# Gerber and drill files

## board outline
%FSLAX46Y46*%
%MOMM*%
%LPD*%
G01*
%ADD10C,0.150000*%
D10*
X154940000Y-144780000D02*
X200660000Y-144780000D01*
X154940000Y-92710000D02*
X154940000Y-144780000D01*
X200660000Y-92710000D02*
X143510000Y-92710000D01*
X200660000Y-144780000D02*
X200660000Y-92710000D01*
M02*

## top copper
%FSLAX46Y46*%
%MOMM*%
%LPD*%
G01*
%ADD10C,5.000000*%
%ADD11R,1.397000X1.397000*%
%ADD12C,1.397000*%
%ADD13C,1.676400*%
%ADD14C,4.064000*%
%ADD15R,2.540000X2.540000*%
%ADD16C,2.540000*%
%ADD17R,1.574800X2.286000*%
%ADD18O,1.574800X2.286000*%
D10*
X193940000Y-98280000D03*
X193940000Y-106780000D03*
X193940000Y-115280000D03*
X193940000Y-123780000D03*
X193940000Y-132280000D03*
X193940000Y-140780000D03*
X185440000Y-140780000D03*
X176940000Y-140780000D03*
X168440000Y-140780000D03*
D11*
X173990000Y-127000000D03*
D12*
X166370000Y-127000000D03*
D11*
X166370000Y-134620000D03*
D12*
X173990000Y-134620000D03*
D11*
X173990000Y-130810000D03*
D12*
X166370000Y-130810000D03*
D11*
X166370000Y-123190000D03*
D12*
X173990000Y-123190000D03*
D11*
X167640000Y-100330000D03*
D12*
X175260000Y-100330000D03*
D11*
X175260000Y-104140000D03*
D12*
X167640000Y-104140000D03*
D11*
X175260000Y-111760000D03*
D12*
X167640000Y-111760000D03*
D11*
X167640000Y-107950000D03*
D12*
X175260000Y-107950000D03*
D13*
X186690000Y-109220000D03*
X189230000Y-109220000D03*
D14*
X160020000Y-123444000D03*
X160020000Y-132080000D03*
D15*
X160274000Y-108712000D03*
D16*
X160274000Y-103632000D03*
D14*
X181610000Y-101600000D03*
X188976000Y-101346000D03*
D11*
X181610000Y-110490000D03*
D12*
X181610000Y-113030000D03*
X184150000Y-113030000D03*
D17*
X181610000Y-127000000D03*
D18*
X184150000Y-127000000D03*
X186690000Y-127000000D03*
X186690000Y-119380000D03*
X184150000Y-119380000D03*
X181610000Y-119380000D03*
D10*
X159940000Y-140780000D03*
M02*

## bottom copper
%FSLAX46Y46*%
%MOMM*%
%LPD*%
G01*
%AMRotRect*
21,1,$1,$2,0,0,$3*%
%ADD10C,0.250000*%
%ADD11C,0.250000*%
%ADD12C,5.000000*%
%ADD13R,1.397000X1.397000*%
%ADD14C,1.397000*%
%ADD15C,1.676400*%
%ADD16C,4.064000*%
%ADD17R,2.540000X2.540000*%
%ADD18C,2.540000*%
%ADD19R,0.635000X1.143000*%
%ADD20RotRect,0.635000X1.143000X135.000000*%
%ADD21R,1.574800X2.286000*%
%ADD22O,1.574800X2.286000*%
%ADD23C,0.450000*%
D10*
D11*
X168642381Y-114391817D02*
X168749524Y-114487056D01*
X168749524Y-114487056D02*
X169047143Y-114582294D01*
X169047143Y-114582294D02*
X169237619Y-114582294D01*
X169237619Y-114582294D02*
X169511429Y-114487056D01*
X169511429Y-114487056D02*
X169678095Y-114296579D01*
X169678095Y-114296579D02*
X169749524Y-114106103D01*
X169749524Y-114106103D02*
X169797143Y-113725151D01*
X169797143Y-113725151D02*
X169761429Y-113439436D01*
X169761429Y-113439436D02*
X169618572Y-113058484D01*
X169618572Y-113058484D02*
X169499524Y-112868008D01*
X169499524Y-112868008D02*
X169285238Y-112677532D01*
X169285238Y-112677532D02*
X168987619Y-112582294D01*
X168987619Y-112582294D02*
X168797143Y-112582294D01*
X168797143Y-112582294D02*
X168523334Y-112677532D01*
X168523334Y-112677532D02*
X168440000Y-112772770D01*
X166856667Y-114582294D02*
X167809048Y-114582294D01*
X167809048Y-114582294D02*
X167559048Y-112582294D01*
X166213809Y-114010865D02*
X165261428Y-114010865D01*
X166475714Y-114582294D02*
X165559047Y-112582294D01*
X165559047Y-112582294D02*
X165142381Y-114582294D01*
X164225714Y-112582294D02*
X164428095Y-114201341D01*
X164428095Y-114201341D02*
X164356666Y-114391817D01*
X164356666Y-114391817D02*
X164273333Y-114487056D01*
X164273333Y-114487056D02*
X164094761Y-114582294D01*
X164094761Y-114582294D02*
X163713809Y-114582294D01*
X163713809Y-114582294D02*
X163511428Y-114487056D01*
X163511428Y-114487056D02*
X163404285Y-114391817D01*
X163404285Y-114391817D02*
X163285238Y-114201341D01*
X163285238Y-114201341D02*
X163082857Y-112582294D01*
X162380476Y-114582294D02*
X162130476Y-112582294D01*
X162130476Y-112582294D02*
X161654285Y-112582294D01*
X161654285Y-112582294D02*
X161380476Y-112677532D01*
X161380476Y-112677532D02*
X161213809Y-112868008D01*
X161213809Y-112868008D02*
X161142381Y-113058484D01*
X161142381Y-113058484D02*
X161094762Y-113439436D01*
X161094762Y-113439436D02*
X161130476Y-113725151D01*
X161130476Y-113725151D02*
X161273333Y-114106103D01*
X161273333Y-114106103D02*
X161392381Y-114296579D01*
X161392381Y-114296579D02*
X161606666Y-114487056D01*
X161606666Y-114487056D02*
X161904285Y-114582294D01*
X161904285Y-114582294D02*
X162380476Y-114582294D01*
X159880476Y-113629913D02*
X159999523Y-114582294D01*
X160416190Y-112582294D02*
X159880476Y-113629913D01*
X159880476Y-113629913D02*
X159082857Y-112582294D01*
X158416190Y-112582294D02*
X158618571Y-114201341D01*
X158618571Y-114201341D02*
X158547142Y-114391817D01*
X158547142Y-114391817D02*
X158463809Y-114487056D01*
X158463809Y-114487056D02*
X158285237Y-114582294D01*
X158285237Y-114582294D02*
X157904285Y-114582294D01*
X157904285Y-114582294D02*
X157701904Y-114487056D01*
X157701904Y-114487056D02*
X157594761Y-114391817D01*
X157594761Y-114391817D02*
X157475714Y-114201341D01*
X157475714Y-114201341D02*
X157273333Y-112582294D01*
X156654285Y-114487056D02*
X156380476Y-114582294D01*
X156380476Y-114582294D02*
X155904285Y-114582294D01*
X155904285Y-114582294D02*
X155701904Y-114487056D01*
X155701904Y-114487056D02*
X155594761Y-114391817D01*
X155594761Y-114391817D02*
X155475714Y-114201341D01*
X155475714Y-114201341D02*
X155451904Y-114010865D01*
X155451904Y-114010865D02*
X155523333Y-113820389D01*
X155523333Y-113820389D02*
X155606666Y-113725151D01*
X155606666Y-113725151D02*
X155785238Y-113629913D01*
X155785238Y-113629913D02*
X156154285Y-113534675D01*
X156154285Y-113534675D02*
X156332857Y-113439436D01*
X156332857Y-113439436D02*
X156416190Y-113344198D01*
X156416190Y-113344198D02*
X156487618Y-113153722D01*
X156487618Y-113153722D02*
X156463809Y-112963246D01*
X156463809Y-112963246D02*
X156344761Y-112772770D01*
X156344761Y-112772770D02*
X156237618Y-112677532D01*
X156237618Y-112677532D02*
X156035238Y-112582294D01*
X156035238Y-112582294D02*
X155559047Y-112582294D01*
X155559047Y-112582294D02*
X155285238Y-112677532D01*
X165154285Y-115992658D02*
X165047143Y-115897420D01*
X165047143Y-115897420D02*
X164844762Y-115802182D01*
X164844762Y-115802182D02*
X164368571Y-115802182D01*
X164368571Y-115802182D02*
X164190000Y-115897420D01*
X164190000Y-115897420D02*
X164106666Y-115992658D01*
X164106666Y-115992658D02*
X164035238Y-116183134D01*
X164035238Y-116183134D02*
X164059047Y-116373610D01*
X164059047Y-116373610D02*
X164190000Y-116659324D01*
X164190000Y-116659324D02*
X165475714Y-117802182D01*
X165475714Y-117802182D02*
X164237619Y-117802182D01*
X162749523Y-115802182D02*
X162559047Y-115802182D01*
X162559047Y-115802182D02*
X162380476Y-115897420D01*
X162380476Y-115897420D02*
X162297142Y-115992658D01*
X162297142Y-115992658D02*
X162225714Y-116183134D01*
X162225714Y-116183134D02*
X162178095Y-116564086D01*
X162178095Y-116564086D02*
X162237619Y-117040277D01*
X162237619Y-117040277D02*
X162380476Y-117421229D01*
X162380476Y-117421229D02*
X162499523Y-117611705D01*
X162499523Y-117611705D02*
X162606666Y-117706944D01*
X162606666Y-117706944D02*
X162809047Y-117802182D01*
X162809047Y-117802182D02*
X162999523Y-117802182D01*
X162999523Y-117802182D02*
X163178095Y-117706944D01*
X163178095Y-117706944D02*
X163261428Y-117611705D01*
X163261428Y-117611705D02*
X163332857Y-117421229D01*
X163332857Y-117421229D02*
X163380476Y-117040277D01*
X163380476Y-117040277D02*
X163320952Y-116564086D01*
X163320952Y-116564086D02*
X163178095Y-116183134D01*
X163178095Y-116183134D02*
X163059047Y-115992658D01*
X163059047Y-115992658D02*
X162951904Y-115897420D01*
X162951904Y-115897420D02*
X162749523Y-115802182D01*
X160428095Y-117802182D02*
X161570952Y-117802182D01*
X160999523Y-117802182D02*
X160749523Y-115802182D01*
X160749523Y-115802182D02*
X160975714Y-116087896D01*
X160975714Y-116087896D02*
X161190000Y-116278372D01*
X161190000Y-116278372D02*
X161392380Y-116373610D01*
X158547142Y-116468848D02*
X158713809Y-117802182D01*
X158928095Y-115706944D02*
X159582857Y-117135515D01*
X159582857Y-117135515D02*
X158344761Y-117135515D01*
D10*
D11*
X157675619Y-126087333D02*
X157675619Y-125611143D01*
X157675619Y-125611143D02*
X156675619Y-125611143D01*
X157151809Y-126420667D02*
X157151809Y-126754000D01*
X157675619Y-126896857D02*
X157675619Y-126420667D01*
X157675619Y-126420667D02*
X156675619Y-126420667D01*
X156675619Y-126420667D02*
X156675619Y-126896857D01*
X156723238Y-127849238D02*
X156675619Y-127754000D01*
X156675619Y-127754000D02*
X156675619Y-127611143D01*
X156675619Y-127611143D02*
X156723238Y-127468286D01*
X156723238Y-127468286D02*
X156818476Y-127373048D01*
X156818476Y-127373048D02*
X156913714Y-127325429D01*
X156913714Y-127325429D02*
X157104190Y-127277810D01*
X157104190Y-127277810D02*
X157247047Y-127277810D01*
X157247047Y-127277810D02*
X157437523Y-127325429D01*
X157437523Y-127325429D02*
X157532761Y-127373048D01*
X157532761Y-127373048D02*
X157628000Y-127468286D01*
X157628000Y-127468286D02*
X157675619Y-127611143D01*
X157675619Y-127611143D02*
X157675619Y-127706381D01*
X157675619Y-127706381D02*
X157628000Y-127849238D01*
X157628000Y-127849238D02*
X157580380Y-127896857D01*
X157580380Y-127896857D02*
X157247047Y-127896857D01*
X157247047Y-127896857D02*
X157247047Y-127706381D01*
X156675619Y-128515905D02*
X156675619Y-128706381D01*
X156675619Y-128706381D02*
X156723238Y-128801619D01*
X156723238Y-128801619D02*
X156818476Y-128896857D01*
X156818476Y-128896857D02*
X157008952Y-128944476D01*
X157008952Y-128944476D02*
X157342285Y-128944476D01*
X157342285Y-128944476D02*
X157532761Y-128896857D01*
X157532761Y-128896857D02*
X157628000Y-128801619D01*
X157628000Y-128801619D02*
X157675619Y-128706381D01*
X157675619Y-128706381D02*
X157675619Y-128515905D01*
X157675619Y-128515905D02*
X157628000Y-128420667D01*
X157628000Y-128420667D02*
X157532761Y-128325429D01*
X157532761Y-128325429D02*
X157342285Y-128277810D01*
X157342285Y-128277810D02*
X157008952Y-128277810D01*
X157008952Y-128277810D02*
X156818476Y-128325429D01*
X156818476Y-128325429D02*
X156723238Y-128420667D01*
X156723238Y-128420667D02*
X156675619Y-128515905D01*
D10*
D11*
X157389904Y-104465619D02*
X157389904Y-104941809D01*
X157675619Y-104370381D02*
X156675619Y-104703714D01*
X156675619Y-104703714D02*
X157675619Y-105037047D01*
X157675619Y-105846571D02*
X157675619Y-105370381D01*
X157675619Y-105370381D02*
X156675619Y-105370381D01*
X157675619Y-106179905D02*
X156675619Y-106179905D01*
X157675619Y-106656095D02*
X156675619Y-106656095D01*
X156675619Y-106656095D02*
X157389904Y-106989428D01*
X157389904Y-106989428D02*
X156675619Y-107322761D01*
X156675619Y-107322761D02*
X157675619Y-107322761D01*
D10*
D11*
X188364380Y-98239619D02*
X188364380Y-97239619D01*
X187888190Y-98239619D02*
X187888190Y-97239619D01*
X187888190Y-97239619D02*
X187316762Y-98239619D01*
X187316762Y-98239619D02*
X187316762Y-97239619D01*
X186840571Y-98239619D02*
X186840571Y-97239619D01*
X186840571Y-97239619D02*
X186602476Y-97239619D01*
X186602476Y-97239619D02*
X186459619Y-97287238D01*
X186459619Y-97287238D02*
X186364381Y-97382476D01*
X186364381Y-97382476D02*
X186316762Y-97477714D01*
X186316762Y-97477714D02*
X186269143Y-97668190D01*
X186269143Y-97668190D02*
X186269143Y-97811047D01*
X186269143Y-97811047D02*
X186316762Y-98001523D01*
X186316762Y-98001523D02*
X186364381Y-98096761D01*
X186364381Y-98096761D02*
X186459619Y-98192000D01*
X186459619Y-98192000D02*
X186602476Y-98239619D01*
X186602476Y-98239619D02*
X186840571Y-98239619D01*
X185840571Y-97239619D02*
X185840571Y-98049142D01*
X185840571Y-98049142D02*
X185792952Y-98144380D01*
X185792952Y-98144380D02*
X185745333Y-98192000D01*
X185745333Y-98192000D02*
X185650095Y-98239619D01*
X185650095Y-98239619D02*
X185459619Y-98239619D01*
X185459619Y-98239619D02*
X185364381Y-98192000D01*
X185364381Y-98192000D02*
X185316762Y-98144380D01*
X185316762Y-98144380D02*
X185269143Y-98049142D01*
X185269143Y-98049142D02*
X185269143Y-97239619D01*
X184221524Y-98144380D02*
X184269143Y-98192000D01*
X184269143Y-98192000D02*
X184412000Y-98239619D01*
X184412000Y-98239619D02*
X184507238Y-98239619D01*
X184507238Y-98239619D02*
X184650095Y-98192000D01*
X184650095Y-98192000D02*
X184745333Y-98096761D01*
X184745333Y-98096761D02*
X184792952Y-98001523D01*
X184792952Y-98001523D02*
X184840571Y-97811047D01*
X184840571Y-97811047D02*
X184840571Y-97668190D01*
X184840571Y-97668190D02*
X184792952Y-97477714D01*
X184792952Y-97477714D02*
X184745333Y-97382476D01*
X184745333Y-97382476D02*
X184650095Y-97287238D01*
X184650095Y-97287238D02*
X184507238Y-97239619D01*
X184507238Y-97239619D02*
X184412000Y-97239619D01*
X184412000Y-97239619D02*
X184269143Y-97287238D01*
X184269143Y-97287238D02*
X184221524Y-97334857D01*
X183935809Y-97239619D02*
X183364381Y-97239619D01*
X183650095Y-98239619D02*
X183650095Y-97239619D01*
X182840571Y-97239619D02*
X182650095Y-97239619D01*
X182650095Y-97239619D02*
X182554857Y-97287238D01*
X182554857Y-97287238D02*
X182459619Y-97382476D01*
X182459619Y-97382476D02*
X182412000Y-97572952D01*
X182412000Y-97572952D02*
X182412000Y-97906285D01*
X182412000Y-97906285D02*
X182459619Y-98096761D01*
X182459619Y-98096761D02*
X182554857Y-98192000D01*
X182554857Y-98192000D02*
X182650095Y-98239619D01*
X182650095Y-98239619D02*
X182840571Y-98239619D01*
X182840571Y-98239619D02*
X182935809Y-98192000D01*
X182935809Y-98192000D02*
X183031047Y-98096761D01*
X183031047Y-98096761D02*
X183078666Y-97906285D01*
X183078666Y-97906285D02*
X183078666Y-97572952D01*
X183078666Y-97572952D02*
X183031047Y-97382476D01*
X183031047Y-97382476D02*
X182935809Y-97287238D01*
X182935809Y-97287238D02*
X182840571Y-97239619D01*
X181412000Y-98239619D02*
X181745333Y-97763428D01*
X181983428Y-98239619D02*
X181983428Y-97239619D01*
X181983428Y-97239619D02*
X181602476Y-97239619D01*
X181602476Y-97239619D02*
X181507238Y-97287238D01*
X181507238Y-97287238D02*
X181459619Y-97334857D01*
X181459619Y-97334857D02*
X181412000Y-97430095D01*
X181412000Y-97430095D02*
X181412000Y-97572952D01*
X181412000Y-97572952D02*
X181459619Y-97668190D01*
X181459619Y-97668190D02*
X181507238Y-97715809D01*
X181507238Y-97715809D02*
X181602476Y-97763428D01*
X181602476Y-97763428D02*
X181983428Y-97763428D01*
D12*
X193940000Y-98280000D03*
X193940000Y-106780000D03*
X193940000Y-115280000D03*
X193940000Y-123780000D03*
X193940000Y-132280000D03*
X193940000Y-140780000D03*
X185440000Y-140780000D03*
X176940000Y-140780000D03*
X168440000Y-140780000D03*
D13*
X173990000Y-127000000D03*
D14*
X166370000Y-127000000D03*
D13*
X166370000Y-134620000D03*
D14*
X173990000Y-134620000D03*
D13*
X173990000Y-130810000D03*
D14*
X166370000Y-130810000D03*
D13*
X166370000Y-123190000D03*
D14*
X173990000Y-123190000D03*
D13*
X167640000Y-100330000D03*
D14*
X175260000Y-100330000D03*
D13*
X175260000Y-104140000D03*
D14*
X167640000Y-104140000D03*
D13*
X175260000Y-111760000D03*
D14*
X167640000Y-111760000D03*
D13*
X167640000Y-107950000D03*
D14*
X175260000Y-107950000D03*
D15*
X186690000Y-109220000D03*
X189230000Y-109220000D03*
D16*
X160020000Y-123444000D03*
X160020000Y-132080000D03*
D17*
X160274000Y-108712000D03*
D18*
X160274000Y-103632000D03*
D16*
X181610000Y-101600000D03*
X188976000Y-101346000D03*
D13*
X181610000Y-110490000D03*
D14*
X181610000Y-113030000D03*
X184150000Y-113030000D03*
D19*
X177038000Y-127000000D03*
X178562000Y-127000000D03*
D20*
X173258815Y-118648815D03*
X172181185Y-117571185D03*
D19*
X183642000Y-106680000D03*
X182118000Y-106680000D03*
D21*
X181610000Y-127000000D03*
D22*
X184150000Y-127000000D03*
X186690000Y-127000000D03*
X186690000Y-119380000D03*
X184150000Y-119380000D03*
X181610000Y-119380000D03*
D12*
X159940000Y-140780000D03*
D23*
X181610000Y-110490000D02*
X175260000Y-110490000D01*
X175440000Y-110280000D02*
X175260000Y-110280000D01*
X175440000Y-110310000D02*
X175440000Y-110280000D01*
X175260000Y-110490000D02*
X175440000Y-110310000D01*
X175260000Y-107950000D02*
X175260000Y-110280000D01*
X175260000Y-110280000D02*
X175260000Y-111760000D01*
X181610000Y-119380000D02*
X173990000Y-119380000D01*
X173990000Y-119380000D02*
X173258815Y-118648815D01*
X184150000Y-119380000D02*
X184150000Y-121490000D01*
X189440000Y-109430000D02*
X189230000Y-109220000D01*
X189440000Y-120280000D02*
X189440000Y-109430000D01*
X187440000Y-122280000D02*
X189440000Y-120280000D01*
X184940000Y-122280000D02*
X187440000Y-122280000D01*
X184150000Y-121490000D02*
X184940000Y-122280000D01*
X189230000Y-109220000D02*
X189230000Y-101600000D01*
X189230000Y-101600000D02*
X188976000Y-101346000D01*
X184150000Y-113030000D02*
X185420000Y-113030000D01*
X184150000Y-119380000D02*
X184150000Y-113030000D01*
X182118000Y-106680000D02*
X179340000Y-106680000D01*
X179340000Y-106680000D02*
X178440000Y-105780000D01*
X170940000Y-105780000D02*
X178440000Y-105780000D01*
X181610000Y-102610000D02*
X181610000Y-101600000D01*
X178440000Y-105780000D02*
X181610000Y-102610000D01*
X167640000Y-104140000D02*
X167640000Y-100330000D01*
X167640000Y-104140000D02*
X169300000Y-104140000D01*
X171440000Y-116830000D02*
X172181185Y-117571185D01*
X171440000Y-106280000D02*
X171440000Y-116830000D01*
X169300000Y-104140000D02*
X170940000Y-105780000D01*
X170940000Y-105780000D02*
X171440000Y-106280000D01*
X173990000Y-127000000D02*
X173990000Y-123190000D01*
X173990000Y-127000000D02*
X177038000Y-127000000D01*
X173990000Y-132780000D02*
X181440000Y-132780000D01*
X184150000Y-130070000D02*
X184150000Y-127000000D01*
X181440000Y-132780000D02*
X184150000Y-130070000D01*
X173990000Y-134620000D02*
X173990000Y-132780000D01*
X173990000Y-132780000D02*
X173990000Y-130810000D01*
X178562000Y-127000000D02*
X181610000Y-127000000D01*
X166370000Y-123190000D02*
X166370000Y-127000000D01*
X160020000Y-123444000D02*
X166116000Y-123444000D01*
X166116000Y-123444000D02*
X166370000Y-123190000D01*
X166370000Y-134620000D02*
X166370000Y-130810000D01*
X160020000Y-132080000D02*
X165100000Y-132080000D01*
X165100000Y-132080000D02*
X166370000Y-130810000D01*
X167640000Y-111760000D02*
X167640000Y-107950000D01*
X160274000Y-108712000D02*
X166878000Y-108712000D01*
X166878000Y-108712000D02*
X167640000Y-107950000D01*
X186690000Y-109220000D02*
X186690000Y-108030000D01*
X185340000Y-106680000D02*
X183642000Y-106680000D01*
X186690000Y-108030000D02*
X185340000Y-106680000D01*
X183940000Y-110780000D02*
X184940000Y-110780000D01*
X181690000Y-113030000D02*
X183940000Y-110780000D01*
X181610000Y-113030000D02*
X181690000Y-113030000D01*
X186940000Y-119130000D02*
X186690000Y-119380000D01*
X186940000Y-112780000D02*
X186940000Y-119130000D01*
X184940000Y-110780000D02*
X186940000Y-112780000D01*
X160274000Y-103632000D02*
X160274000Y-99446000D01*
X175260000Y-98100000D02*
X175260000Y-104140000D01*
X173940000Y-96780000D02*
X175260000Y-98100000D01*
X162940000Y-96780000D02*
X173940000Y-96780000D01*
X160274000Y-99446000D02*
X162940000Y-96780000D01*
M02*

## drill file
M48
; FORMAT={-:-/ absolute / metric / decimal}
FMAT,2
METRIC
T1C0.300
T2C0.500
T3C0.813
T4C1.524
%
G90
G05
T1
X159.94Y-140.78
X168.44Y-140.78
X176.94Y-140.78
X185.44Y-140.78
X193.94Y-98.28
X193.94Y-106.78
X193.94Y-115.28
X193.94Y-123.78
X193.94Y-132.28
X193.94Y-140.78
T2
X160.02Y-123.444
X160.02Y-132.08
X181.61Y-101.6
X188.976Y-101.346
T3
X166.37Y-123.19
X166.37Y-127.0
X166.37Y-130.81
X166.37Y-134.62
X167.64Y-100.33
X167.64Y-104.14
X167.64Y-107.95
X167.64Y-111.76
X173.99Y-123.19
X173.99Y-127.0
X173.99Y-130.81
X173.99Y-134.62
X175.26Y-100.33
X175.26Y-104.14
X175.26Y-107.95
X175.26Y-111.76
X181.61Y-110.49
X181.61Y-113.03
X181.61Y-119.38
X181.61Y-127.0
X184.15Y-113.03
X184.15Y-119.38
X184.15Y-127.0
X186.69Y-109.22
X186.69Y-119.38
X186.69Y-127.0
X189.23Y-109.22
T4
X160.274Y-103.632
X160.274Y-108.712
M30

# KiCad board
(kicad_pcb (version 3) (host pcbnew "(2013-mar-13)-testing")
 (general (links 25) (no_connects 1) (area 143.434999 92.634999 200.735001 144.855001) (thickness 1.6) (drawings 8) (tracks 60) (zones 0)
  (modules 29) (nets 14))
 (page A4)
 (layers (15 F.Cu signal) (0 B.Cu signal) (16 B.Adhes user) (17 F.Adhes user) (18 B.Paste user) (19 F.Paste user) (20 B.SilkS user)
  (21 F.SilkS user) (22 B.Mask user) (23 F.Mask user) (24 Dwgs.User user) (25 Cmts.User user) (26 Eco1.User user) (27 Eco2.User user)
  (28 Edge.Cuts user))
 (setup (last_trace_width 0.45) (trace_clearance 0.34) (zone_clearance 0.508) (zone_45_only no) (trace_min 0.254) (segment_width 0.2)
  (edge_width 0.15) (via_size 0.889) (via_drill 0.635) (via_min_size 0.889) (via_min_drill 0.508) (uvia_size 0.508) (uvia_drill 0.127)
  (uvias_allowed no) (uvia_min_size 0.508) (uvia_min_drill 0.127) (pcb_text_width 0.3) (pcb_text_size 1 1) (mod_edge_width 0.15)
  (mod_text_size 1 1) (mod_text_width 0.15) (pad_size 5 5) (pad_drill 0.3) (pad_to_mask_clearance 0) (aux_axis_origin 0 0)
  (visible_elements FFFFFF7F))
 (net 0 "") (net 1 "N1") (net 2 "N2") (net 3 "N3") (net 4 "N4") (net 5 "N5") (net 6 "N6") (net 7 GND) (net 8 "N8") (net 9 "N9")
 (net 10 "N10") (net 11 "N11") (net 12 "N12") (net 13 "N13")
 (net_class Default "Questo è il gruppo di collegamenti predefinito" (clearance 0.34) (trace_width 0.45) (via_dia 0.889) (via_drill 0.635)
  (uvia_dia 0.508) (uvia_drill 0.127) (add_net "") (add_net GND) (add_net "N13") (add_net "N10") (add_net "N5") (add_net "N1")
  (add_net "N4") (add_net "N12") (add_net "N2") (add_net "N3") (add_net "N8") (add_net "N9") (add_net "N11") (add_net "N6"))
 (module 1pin (layer F.Cu) (at 193.94 98.28)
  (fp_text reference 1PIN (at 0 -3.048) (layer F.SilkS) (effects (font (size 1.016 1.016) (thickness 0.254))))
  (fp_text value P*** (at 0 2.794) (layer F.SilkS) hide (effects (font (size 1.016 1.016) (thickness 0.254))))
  (pad 1 thru_hole circle (at 0 0) (size 5 5) (drill 0.3) (layers *.Cu *.Mask F.SilkS)))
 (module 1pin (layer F.Cu) (at 193.94 106.78)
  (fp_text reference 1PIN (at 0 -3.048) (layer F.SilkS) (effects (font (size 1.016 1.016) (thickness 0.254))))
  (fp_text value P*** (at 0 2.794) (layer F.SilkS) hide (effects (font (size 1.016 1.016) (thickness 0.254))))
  (pad 1 thru_hole circle (at 0 0) (size 5 5) (drill 0.3) (layers *.Cu *.Mask F.SilkS)))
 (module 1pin (layer F.Cu) (at 193.94 115.28)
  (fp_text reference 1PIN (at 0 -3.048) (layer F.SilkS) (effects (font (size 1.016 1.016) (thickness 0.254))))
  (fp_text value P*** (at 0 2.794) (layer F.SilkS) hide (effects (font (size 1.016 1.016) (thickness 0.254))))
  (pad 1 thru_hole circle (at 0 0) (size 5 5) (drill 0.3) (layers *.Cu *.Mask F.SilkS)))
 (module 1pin (layer F.Cu) (at 193.94 123.78)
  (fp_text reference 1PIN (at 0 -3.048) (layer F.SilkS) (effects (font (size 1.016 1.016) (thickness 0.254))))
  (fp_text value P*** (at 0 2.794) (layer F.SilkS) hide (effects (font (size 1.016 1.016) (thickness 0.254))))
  (pad 1 thru_hole circle (at 0 0) (size 5 5) (drill 0.3) (layers *.Cu *.Mask F.SilkS)))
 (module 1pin (layer F.Cu) (at 193.94 132.28)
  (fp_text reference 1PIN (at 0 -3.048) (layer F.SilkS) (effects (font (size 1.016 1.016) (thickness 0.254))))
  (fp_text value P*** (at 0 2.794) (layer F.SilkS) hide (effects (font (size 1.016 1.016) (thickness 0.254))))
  (pad 1 thru_hole circle (at 0 0) (size 5 5) (drill 0.3) (layers *.Cu *.Mask F.SilkS)))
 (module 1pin (layer F.Cu) (at 193.94 140.78)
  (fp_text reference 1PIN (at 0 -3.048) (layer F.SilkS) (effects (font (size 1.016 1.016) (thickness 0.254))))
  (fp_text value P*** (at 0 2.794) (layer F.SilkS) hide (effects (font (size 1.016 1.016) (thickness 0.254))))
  (pad 1 thru_hole circle (at 0 0) (size 5 5) (drill 0.3) (layers *.Cu *.Mask F.SilkS)))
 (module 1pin (layer F.Cu) (at 185.44 140.78)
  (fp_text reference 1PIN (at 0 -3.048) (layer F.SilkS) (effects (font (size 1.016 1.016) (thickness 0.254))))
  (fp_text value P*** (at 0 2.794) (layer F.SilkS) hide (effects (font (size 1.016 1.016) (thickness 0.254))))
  (pad 1 thru_hole circle (at 0 0) (size 5 5) (drill 0.3) (layers *.Cu *.Mask F.SilkS)))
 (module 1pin (layer F.Cu) (at 176.94 140.78)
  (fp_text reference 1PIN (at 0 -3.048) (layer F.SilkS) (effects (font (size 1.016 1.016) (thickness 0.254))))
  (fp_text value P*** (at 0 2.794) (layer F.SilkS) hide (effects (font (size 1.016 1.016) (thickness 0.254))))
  (pad 1 thru_hole circle (at 0 0) (size 5 5) (drill 0.3) (layers *.Cu *.Mask F.SilkS)))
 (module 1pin (layer F.Cu) (at 168.44 140.78)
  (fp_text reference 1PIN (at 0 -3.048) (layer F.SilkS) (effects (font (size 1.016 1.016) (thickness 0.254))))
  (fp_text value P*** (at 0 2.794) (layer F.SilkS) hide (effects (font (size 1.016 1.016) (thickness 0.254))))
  (pad 1 thru_hole circle (at 0 0) (size 5 5) (drill 0.3) (layers *.Cu *.Mask F.SilkS)))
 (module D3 (layer F.Cu) (at 170.18 127)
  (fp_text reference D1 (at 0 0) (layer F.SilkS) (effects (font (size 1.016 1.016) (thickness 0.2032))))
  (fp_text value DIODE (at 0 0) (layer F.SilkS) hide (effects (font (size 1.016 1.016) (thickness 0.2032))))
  (pad 2 thru_hole rect (at 3.81 0) (size 1.397 1.397) (drill 0.8128) (layers *.Cu *.Mask F.SilkS) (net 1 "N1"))
  (pad 1 thru_hole circle (at -3.81 0) (size 1.397 1.397) (drill 0.8128) (layers *.Cu *.Mask F.SilkS) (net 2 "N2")))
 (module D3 (layer F.Cu) (at 170.18 134.62 180)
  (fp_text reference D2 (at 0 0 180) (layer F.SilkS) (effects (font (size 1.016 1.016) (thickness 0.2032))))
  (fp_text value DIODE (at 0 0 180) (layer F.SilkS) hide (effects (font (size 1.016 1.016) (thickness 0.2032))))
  (pad 2 thru_hole rect (at 3.81 0 180) (size 1.397 1.397) (drill 0.8128) (layers *.Cu *.Mask F.SilkS) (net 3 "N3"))
  (pad 1 thru_hole circle (at -3.81 0 180) (size 1.397 1.397) (drill 0.8128) (layers *.Cu *.Mask F.SilkS) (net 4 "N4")))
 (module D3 (layer F.Cu) (at 170.18 130.81)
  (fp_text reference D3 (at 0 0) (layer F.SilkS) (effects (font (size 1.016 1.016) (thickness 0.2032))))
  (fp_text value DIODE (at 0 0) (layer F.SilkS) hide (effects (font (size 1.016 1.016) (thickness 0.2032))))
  (pad 2 thru_hole rect (at 3.81 0) (size 1.397 1.397) (drill 0.8128) (layers *.Cu *.Mask F.SilkS) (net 4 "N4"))
  (pad 1 thru_hole circle (at -3.81 0) (size 1.397 1.397) (drill 0.8128) (layers *.Cu *.Mask F.SilkS) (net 3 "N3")))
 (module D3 (layer F.Cu) (at 170.18 123.19 180)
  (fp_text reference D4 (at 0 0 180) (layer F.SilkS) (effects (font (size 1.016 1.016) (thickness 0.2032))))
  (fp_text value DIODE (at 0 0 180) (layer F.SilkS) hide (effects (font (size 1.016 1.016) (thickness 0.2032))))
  (pad 2 thru_hole rect (at 3.81 0 180) (size 1.397 1.397) (drill 0.8128) (layers *.Cu *.Mask F.SilkS) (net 2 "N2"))
  (pad 1 thru_hole circle (at -3.81 0 180) (size 1.397 1.397) (drill 0.8128) (layers *.Cu *.Mask F.SilkS) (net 1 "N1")))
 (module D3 (layer F.Cu) (at 171.45 100.33 180)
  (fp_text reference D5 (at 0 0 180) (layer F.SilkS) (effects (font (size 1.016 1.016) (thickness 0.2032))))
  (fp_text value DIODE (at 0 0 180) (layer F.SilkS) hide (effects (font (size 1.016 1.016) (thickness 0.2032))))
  (pad 2 thru_hole rect (at 3.81 0 180) (size 1.397 1.397) (drill 0.8128) (layers *.Cu *.Mask F.SilkS) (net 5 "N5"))
  (pad 1 thru_hole circle (at -3.81 0 180) (size 1.397 1.397) (drill 0.8128) (layers *.Cu *.Mask F.SilkS) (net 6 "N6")))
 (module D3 (layer F.Cu) (at 171.45 104.14)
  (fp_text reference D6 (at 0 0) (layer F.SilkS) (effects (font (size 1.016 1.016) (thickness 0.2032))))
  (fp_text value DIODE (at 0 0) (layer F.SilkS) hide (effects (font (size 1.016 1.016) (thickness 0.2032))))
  (pad 2 thru_hole rect (at 3.81 0) (size 1.397 1.397) (drill 0.8128) (layers *.Cu *.Mask F.SilkS) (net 6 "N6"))
  (pad 1 thru_hole circle (at -3.81 0) (size 1.397 1.397) (drill 0.8128) (layers *.Cu *.Mask F.SilkS) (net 5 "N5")))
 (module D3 (layer F.Cu) (at 171.45 111.76)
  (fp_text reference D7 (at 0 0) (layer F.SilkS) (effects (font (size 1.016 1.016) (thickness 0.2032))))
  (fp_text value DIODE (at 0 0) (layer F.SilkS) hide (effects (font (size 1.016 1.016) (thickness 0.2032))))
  (pad 2 thru_hole rect (at 3.81 0) (size 1.397 1.397) (drill 0.8128) (layers *.Cu *.Mask F.SilkS) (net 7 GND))
  (pad 1 thru_hole circle (at -3.81 0) (size 1.397 1.397) (drill 0.8128) (layers *.Cu *.Mask F.SilkS) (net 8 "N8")))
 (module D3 (layer F.Cu) (at 171.45 107.95 180)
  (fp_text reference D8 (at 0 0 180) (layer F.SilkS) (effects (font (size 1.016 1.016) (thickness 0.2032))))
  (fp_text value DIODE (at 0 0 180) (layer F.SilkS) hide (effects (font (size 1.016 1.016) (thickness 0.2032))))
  (pad 2 thru_hole rect (at 3.81 0 180) (size 1.397 1.397) (drill 0.8128) (layers *.Cu *.Mask F.SilkS) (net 8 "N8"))
  (pad 1 thru_hole circle (at -3.81 0 180) (size 1.397 1.397) (drill 0.8128) (layers *.Cu *.Mask F.SilkS) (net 7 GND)))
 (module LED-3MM (layer F.Cu) (at 187.96 109.22)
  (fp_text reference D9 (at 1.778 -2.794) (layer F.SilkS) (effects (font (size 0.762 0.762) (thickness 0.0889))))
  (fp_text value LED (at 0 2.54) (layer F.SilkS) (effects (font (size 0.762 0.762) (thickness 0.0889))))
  (pad 1 thru_hole circle (at -1.27 0) (size 1.6764 1.6764) (drill 0.8128) (layers *.Cu *.Mask F.SilkS) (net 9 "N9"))
  (pad 2 thru_hole circle (at 1.27 0) (size 1.6764 1.6764) (drill 0.8128) (layers *.Cu *.Mask F.SilkS) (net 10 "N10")))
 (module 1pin (layer F.Cu) (at 160.02 123.444)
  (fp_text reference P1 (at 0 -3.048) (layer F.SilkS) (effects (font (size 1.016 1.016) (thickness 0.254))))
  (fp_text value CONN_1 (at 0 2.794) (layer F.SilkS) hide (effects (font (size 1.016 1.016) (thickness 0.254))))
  (pad 1 thru_hole circle (at 0 0) (size 4.064 4.064) (drill 0.5) (layers *.Cu *.Mask F.SilkS) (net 2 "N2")))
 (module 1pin (layer F.Cu) (at 160.02 132.08)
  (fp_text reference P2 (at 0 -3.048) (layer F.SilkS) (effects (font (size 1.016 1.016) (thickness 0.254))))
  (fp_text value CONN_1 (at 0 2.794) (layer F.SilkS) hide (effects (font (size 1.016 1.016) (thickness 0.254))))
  (pad 1 thru_hole circle (at 0 0) (size 4.064 4.064) (drill 0.5) (layers *.Cu *.Mask F.SilkS) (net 3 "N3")))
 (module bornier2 (layer F.Cu) (at 160.274 106.172 90)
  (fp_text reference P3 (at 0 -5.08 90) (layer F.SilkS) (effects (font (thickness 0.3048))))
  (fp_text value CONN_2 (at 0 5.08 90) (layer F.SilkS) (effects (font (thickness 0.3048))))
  (pad 1 thru_hole rect (at -2.54 0 90) (size 2.54 2.54) (drill 1.524) (layers *.Cu *.Mask F.SilkS) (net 8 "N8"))
  (pad 2 thru_hole circle (at 2.54 0 90) (size 2.54 2.54) (drill 1.524) (layers *.Cu *.Mask F.SilkS) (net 6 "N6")))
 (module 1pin (layer F.Cu) (at 181.61 101.6)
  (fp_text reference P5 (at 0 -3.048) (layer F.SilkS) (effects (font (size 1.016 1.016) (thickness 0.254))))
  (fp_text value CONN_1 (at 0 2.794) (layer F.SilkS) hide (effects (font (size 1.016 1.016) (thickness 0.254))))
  (pad 1 thru_hole circle (at 0 0) (size 4.064 4.064) (drill 0.5) (layers *.Cu *.Mask F.SilkS) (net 5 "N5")))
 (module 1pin (layer F.Cu) (at 188.976 101.346)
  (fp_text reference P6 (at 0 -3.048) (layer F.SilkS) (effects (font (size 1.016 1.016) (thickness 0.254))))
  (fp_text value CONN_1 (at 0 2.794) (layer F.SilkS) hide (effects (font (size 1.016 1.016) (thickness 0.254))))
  (pad 1 thru_hole circle (at 0 0) (size 4.064 4.064) (drill 0.5) (layers *.Cu *.Mask F.SilkS) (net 10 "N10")))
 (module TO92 (layer F.Cu) (at 182.88 111.76 90)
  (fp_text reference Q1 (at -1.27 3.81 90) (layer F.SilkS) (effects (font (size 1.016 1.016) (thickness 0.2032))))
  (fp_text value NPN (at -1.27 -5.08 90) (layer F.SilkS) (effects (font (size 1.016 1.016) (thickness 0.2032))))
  (pad 1 thru_hole rect (at 1.27 -1.27 90) (size 1.397 1.397) (drill 0.8128) (layers *.Cu *.Mask F.SilkS) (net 7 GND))
  (pad 2 thru_hole circle (at -1.27 -1.27 90) (size 1.397 1.397) (drill 0.8128) (layers *.Cu *.Mask F.SilkS) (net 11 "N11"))
  (pad 3 thru_hole circle (at -1.27 1.27 90) (size 1.397 1.397) (drill 0.8128) (layers *.Cu *.Mask F.SilkS) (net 10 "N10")))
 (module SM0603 (layer B.Cu) (at 177.8 127)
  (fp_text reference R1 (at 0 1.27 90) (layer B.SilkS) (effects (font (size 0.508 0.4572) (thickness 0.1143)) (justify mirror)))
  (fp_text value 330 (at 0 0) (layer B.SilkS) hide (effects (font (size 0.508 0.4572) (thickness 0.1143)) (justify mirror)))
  (pad 1 smd rect (at -0.762 0) (size 0.635 1.143) (layers B.Cu B.Paste B.Mask) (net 1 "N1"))
  (pad 2 smd rect (at 0.762 0) (size 0.635 1.143) (layers B.Cu B.Paste B.Mask) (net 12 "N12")))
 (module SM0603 (layer B.Cu) (at 172.72 118.11 135)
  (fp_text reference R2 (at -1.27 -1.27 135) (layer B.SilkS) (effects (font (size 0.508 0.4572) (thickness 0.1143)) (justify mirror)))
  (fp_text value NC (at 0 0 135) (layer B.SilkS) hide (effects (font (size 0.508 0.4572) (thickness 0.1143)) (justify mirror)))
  (pad 1 smd rect (at -0.762 0 135) (size 0.635 1.143) (layers B.Cu B.Paste B.Mask) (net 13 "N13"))
  (pad 2 smd rect (at 0.762 0 135) (size 0.635 1.143) (layers B.Cu B.Paste B.Mask) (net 5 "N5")))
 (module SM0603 (layer B.Cu) (at 182.88 106.68 180)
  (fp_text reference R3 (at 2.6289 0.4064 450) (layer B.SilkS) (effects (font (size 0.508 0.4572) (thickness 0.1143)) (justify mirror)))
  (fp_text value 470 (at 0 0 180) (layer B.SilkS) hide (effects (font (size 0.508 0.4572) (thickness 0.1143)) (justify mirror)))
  (pad 1 smd rect (at -0.762 0 180) (size 0.635 1.143) (layers B.Cu B.Paste B.Mask) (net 9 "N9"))
  (pad 2 smd rect (at 0.762 0 180) (size 0.635 1.143) (layers B.Cu B.Paste B.Mask) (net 5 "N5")))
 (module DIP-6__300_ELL (layer F.Cu) (at 184.15 123.19)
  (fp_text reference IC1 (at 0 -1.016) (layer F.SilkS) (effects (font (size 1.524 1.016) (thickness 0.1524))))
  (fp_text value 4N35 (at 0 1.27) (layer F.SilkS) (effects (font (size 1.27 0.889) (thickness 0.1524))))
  (pad 1 thru_hole rect (at -2.54 3.81) (size 1.5748 2.286) (drill 0.8128) (layers *.Cu *.Mask F.SilkS) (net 12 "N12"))
  (pad 2 thru_hole oval (at 0 3.81) (size 1.5748 2.286) (drill 0.8128) (layers *.Cu *.Mask F.SilkS) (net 4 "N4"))
  (pad 3 thru_hole oval (at 2.54 3.81) (size 1.5748 2.286) (drill 0.8128) (layers *.Cu *.Mask F.SilkS))
  (pad 4 thru_hole oval (at 2.54 -3.81) (size 1.5748 2.286) (drill 0.8128) (layers *.Cu *.Mask F.SilkS) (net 11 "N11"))
  (pad 5 thru_hole oval (at 0 -3.81) (size 1.5748 2.286) (drill 0.8128) (layers *.Cu *.Mask F.SilkS) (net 10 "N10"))
  (pad 6 thru_hole oval (at -2.54 -3.81) (size 1.5748 2.286) (drill 0.8128) (layers *.Cu *.Mask F.SilkS) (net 13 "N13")))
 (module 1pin (layer F.Cu) (at 159.94 140.78)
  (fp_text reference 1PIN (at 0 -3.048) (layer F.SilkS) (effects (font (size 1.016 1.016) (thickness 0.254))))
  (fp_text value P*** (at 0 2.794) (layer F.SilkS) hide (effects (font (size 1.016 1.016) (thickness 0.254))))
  (pad 1 thru_hole circle (at 0 0) (size 5 5) (drill 0.3) (layers *.Cu *.Mask F.SilkS)))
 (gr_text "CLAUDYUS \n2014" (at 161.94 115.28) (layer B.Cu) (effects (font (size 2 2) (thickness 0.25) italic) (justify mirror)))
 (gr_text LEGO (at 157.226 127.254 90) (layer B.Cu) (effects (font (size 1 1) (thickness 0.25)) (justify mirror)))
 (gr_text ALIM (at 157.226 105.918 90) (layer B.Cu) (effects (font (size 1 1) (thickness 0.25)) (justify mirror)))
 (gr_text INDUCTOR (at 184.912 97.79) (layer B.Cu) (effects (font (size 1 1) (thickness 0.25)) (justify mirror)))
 (gr_line (start 154.94 144.78) (end 200.66 144.78) (angle 90) (layer Edge.Cuts) (width 0.15))
 (gr_line (start 154.94 92.71) (end 154.94 144.78) (angle 90) (layer Edge.Cuts) (width 0.15))
 (gr_line (start 200.66 92.71) (end 143.51 92.71) (angle 90) (layer Edge.Cuts) (width 0.15))
 (gr_line (start 200.66 144.78) (end 200.66 92.71) (angle 90) (layer Edge.Cuts) (width 0.15))
 (segment (start 181.61 110.49) (end 175.26 110.49) (width 0.45) (layer B.Cu) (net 7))
 (segment (start 175.44 110.28) (end 175.26 110.28) (width 0.45) (layer B.Cu) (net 7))
 (segment (start 175.44 110.31) (end 175.44 110.28) (width 0.45) (layer B.Cu) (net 7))
 (segment (start 175.26 110.49) (end 175.44 110.31) (width 0.45) (layer B.Cu) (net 7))
 (segment (start 175.26 107.95) (end 175.26 110.28) (width 0.45) (layer B.Cu) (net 7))
 (segment (start 175.26 110.28) (end 175.26 111.76) (width 0.45) (layer B.Cu) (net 7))
 (segment (start 181.61 119.38) (end 173.99 119.38) (width 0.45) (layer B.Cu) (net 13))
 (segment (start 173.99 119.38) (end 173.258815 118.648815) (width 0.45) (layer B.Cu) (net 13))
 (segment (start 184.15 119.38) (end 184.15 121.49) (width 0.45) (layer B.Cu) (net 10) (status 400000))
 (segment (start 189.44 109.43) (end 189.23 109.22) (width 0.45) (layer B.Cu) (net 10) (status C00000))
 (segment (start 189.44 120.28) (end 189.44 109.43) (width 0.45) (layer B.Cu) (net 10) (status 800000))
 (segment (start 187.44 122.28) (end 189.44 120.28) (width 0.45) (layer B.Cu) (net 10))
 (segment (start 184.94 122.28) (end 187.44 122.28) (width 0.45) (layer B.Cu) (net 10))
 (segment (start 184.15 121.49) (end 184.94 122.28) (width 0.45) (layer B.Cu) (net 10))
 (segment (start 189.23 109.22) (end 189.23 101.6) (width 0.45) (layer B.Cu) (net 10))
 (segment (start 189.23 101.6) (end 188.976 101.346) (width 0.45) (layer B.Cu) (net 10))
 (segment (start 184.15 113.03) (end 185.42 113.03) (width 0.45) (layer B.Cu) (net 10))
 (segment (start 184.15 119.38) (end 184.15 113.03) (width 0.45) (layer B.Cu) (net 10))
 (segment (start 182.118 106.68) (end 179.34 106.68) (width 0.45) (layer B.Cu) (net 5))
 (segment (start 179.34 106.68) (end 178.44 105.78) (width 0.45) (layer B.Cu) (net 5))
 (segment (start 170.94 105.78) (end 178.44 105.78) (width 0.45) (layer B.Cu) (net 5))
 (segment (start 181.61 102.61) (end 181.61 101.6) (width 0.45) (layer B.Cu) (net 5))
 (segment (start 178.44 105.78) (end 181.61 102.61) (width 0.45) (layer B.Cu) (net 5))
 (segment (start 167.64 104.14) (end 167.64 100.33) (width 0.45) (layer B.Cu) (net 5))
 (segment (start 167.64 104.14) (end 169.3 104.14) (width 0.45) (layer B.Cu) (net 5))
 (segment (start 171.44 116.83) (end 172.181185 117.571185) (width 0.45) (layer B.Cu) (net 5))
 (segment (start 171.44 106.28) (end 171.44 116.83) (width 0.45) (layer B.Cu) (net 5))
 (segment (start 169.3 104.14) (end 170.94 105.78) (width 0.45) (layer B.Cu) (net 5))
 (segment (start 170.94 105.78) (end 171.44 106.28) (width 0.45) (layer B.Cu) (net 5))
 (segment (start 173.99 127) (end 173.99 123.19) (width 0.45) (layer B.Cu) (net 1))
 (segment (start 173.99 127) (end 177.038 127) (width 0.45) (layer B.Cu) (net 1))
 (segment (start 173.99 132.78) (end 181.44 132.78) (width 0.45) (layer B.Cu) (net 4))
 (segment (start 184.15 130.07) (end 184.15 127) (width 0.45) (layer B.Cu) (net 4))
 (segment (start 181.44 132.78) (end 184.15 130.07) (width 0.45) (layer B.Cu) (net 4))
 (segment (start 173.99 134.62) (end 173.99 132.78) (width 0.45) (layer B.Cu) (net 4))
 (segment (start 173.99 132.78) (end 173.99 130.81) (width 0.45) (layer B.Cu) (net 4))
 (segment (start 178.562 127) (end 181.61 127) (width 0.45) (layer B.Cu) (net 12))
 (segment (start 166.37 123.19) (end 166.37 127) (width 0.45) (layer B.Cu) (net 2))
 (segment (start 160.02 123.444) (end 166.116 123.444) (width 0.45) (layer B.Cu) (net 2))
 (segment (start 166.116 123.444) (end 166.37 123.19) (width 0.45) (layer B.Cu) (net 2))
 (segment (start 166.37 134.62) (end 166.37 130.81) (width 0.45) (layer B.Cu) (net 3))
 (segment (start 160.02 132.08) (end 165.1 132.08) (width 0.45) (layer B.Cu) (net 3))
 (segment (start 165.1 132.08) (end 166.37 130.81) (width 0.45) (layer B.Cu) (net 3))
 (segment (start 167.64 111.76) (end 167.64 107.95) (width 0.45) (layer B.Cu) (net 8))
 (segment (start 160.274 108.712) (end 166.878 108.712) (width 0.45) (layer B.Cu) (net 8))
 (segment (start 166.878 108.712) (end 167.64 107.95) (width 0.45) (layer B.Cu) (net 8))
 (segment (start 186.69 109.22) (end 186.69 108.03) (width 0.45) (layer B.Cu) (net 9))
 (segment (start 185.34 106.68) (end 183.642 106.68) (width 0.45) (layer B.Cu) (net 9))
 (segment (start 186.69 108.03) (end 185.34 106.68) (width 0.45) (layer B.Cu) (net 9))
 (segment (start 183.94 110.78) (end 184.94 110.78) (width 0.45) (layer B.Cu) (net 11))
 (segment (start 181.69 113.03) (end 183.94 110.78) (width 0.45) (layer B.Cu) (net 11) (status 400000))
 (segment (start 181.61 113.03) (end 181.69 113.03) (width 0.45) (layer B.Cu) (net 11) (status C00000))
 (segment (start 186.94 119.13) (end 186.69 119.38) (width 0.45) (layer B.Cu) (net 11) (status C00000))
 (segment (start 186.94 112.78) (end 186.94 119.13) (width 0.45) (layer B.Cu) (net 11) (status 800000))
 (segment (start 184.94 110.78) (end 186.94 112.78) (width 0.45) (layer B.Cu) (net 11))
 (segment (start 160.274 103.632) (end 160.274 99.446) (width 0.45) (layer B.Cu) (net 6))
 (segment (start 175.26 98.1) (end 175.26 104.14) (width 0.45) (layer B.Cu) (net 6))
 (segment (start 173.94 96.78) (end 175.26 98.1) (width 0.45) (layer B.Cu) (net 6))
 (segment (start 162.94 96.78) (end 173.94 96.78) (width 0.45) (layer B.Cu) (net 6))
 (segment (start 160.274 99.446) (end 162.94 96.78) (width 0.45) (layer B.Cu) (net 6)))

